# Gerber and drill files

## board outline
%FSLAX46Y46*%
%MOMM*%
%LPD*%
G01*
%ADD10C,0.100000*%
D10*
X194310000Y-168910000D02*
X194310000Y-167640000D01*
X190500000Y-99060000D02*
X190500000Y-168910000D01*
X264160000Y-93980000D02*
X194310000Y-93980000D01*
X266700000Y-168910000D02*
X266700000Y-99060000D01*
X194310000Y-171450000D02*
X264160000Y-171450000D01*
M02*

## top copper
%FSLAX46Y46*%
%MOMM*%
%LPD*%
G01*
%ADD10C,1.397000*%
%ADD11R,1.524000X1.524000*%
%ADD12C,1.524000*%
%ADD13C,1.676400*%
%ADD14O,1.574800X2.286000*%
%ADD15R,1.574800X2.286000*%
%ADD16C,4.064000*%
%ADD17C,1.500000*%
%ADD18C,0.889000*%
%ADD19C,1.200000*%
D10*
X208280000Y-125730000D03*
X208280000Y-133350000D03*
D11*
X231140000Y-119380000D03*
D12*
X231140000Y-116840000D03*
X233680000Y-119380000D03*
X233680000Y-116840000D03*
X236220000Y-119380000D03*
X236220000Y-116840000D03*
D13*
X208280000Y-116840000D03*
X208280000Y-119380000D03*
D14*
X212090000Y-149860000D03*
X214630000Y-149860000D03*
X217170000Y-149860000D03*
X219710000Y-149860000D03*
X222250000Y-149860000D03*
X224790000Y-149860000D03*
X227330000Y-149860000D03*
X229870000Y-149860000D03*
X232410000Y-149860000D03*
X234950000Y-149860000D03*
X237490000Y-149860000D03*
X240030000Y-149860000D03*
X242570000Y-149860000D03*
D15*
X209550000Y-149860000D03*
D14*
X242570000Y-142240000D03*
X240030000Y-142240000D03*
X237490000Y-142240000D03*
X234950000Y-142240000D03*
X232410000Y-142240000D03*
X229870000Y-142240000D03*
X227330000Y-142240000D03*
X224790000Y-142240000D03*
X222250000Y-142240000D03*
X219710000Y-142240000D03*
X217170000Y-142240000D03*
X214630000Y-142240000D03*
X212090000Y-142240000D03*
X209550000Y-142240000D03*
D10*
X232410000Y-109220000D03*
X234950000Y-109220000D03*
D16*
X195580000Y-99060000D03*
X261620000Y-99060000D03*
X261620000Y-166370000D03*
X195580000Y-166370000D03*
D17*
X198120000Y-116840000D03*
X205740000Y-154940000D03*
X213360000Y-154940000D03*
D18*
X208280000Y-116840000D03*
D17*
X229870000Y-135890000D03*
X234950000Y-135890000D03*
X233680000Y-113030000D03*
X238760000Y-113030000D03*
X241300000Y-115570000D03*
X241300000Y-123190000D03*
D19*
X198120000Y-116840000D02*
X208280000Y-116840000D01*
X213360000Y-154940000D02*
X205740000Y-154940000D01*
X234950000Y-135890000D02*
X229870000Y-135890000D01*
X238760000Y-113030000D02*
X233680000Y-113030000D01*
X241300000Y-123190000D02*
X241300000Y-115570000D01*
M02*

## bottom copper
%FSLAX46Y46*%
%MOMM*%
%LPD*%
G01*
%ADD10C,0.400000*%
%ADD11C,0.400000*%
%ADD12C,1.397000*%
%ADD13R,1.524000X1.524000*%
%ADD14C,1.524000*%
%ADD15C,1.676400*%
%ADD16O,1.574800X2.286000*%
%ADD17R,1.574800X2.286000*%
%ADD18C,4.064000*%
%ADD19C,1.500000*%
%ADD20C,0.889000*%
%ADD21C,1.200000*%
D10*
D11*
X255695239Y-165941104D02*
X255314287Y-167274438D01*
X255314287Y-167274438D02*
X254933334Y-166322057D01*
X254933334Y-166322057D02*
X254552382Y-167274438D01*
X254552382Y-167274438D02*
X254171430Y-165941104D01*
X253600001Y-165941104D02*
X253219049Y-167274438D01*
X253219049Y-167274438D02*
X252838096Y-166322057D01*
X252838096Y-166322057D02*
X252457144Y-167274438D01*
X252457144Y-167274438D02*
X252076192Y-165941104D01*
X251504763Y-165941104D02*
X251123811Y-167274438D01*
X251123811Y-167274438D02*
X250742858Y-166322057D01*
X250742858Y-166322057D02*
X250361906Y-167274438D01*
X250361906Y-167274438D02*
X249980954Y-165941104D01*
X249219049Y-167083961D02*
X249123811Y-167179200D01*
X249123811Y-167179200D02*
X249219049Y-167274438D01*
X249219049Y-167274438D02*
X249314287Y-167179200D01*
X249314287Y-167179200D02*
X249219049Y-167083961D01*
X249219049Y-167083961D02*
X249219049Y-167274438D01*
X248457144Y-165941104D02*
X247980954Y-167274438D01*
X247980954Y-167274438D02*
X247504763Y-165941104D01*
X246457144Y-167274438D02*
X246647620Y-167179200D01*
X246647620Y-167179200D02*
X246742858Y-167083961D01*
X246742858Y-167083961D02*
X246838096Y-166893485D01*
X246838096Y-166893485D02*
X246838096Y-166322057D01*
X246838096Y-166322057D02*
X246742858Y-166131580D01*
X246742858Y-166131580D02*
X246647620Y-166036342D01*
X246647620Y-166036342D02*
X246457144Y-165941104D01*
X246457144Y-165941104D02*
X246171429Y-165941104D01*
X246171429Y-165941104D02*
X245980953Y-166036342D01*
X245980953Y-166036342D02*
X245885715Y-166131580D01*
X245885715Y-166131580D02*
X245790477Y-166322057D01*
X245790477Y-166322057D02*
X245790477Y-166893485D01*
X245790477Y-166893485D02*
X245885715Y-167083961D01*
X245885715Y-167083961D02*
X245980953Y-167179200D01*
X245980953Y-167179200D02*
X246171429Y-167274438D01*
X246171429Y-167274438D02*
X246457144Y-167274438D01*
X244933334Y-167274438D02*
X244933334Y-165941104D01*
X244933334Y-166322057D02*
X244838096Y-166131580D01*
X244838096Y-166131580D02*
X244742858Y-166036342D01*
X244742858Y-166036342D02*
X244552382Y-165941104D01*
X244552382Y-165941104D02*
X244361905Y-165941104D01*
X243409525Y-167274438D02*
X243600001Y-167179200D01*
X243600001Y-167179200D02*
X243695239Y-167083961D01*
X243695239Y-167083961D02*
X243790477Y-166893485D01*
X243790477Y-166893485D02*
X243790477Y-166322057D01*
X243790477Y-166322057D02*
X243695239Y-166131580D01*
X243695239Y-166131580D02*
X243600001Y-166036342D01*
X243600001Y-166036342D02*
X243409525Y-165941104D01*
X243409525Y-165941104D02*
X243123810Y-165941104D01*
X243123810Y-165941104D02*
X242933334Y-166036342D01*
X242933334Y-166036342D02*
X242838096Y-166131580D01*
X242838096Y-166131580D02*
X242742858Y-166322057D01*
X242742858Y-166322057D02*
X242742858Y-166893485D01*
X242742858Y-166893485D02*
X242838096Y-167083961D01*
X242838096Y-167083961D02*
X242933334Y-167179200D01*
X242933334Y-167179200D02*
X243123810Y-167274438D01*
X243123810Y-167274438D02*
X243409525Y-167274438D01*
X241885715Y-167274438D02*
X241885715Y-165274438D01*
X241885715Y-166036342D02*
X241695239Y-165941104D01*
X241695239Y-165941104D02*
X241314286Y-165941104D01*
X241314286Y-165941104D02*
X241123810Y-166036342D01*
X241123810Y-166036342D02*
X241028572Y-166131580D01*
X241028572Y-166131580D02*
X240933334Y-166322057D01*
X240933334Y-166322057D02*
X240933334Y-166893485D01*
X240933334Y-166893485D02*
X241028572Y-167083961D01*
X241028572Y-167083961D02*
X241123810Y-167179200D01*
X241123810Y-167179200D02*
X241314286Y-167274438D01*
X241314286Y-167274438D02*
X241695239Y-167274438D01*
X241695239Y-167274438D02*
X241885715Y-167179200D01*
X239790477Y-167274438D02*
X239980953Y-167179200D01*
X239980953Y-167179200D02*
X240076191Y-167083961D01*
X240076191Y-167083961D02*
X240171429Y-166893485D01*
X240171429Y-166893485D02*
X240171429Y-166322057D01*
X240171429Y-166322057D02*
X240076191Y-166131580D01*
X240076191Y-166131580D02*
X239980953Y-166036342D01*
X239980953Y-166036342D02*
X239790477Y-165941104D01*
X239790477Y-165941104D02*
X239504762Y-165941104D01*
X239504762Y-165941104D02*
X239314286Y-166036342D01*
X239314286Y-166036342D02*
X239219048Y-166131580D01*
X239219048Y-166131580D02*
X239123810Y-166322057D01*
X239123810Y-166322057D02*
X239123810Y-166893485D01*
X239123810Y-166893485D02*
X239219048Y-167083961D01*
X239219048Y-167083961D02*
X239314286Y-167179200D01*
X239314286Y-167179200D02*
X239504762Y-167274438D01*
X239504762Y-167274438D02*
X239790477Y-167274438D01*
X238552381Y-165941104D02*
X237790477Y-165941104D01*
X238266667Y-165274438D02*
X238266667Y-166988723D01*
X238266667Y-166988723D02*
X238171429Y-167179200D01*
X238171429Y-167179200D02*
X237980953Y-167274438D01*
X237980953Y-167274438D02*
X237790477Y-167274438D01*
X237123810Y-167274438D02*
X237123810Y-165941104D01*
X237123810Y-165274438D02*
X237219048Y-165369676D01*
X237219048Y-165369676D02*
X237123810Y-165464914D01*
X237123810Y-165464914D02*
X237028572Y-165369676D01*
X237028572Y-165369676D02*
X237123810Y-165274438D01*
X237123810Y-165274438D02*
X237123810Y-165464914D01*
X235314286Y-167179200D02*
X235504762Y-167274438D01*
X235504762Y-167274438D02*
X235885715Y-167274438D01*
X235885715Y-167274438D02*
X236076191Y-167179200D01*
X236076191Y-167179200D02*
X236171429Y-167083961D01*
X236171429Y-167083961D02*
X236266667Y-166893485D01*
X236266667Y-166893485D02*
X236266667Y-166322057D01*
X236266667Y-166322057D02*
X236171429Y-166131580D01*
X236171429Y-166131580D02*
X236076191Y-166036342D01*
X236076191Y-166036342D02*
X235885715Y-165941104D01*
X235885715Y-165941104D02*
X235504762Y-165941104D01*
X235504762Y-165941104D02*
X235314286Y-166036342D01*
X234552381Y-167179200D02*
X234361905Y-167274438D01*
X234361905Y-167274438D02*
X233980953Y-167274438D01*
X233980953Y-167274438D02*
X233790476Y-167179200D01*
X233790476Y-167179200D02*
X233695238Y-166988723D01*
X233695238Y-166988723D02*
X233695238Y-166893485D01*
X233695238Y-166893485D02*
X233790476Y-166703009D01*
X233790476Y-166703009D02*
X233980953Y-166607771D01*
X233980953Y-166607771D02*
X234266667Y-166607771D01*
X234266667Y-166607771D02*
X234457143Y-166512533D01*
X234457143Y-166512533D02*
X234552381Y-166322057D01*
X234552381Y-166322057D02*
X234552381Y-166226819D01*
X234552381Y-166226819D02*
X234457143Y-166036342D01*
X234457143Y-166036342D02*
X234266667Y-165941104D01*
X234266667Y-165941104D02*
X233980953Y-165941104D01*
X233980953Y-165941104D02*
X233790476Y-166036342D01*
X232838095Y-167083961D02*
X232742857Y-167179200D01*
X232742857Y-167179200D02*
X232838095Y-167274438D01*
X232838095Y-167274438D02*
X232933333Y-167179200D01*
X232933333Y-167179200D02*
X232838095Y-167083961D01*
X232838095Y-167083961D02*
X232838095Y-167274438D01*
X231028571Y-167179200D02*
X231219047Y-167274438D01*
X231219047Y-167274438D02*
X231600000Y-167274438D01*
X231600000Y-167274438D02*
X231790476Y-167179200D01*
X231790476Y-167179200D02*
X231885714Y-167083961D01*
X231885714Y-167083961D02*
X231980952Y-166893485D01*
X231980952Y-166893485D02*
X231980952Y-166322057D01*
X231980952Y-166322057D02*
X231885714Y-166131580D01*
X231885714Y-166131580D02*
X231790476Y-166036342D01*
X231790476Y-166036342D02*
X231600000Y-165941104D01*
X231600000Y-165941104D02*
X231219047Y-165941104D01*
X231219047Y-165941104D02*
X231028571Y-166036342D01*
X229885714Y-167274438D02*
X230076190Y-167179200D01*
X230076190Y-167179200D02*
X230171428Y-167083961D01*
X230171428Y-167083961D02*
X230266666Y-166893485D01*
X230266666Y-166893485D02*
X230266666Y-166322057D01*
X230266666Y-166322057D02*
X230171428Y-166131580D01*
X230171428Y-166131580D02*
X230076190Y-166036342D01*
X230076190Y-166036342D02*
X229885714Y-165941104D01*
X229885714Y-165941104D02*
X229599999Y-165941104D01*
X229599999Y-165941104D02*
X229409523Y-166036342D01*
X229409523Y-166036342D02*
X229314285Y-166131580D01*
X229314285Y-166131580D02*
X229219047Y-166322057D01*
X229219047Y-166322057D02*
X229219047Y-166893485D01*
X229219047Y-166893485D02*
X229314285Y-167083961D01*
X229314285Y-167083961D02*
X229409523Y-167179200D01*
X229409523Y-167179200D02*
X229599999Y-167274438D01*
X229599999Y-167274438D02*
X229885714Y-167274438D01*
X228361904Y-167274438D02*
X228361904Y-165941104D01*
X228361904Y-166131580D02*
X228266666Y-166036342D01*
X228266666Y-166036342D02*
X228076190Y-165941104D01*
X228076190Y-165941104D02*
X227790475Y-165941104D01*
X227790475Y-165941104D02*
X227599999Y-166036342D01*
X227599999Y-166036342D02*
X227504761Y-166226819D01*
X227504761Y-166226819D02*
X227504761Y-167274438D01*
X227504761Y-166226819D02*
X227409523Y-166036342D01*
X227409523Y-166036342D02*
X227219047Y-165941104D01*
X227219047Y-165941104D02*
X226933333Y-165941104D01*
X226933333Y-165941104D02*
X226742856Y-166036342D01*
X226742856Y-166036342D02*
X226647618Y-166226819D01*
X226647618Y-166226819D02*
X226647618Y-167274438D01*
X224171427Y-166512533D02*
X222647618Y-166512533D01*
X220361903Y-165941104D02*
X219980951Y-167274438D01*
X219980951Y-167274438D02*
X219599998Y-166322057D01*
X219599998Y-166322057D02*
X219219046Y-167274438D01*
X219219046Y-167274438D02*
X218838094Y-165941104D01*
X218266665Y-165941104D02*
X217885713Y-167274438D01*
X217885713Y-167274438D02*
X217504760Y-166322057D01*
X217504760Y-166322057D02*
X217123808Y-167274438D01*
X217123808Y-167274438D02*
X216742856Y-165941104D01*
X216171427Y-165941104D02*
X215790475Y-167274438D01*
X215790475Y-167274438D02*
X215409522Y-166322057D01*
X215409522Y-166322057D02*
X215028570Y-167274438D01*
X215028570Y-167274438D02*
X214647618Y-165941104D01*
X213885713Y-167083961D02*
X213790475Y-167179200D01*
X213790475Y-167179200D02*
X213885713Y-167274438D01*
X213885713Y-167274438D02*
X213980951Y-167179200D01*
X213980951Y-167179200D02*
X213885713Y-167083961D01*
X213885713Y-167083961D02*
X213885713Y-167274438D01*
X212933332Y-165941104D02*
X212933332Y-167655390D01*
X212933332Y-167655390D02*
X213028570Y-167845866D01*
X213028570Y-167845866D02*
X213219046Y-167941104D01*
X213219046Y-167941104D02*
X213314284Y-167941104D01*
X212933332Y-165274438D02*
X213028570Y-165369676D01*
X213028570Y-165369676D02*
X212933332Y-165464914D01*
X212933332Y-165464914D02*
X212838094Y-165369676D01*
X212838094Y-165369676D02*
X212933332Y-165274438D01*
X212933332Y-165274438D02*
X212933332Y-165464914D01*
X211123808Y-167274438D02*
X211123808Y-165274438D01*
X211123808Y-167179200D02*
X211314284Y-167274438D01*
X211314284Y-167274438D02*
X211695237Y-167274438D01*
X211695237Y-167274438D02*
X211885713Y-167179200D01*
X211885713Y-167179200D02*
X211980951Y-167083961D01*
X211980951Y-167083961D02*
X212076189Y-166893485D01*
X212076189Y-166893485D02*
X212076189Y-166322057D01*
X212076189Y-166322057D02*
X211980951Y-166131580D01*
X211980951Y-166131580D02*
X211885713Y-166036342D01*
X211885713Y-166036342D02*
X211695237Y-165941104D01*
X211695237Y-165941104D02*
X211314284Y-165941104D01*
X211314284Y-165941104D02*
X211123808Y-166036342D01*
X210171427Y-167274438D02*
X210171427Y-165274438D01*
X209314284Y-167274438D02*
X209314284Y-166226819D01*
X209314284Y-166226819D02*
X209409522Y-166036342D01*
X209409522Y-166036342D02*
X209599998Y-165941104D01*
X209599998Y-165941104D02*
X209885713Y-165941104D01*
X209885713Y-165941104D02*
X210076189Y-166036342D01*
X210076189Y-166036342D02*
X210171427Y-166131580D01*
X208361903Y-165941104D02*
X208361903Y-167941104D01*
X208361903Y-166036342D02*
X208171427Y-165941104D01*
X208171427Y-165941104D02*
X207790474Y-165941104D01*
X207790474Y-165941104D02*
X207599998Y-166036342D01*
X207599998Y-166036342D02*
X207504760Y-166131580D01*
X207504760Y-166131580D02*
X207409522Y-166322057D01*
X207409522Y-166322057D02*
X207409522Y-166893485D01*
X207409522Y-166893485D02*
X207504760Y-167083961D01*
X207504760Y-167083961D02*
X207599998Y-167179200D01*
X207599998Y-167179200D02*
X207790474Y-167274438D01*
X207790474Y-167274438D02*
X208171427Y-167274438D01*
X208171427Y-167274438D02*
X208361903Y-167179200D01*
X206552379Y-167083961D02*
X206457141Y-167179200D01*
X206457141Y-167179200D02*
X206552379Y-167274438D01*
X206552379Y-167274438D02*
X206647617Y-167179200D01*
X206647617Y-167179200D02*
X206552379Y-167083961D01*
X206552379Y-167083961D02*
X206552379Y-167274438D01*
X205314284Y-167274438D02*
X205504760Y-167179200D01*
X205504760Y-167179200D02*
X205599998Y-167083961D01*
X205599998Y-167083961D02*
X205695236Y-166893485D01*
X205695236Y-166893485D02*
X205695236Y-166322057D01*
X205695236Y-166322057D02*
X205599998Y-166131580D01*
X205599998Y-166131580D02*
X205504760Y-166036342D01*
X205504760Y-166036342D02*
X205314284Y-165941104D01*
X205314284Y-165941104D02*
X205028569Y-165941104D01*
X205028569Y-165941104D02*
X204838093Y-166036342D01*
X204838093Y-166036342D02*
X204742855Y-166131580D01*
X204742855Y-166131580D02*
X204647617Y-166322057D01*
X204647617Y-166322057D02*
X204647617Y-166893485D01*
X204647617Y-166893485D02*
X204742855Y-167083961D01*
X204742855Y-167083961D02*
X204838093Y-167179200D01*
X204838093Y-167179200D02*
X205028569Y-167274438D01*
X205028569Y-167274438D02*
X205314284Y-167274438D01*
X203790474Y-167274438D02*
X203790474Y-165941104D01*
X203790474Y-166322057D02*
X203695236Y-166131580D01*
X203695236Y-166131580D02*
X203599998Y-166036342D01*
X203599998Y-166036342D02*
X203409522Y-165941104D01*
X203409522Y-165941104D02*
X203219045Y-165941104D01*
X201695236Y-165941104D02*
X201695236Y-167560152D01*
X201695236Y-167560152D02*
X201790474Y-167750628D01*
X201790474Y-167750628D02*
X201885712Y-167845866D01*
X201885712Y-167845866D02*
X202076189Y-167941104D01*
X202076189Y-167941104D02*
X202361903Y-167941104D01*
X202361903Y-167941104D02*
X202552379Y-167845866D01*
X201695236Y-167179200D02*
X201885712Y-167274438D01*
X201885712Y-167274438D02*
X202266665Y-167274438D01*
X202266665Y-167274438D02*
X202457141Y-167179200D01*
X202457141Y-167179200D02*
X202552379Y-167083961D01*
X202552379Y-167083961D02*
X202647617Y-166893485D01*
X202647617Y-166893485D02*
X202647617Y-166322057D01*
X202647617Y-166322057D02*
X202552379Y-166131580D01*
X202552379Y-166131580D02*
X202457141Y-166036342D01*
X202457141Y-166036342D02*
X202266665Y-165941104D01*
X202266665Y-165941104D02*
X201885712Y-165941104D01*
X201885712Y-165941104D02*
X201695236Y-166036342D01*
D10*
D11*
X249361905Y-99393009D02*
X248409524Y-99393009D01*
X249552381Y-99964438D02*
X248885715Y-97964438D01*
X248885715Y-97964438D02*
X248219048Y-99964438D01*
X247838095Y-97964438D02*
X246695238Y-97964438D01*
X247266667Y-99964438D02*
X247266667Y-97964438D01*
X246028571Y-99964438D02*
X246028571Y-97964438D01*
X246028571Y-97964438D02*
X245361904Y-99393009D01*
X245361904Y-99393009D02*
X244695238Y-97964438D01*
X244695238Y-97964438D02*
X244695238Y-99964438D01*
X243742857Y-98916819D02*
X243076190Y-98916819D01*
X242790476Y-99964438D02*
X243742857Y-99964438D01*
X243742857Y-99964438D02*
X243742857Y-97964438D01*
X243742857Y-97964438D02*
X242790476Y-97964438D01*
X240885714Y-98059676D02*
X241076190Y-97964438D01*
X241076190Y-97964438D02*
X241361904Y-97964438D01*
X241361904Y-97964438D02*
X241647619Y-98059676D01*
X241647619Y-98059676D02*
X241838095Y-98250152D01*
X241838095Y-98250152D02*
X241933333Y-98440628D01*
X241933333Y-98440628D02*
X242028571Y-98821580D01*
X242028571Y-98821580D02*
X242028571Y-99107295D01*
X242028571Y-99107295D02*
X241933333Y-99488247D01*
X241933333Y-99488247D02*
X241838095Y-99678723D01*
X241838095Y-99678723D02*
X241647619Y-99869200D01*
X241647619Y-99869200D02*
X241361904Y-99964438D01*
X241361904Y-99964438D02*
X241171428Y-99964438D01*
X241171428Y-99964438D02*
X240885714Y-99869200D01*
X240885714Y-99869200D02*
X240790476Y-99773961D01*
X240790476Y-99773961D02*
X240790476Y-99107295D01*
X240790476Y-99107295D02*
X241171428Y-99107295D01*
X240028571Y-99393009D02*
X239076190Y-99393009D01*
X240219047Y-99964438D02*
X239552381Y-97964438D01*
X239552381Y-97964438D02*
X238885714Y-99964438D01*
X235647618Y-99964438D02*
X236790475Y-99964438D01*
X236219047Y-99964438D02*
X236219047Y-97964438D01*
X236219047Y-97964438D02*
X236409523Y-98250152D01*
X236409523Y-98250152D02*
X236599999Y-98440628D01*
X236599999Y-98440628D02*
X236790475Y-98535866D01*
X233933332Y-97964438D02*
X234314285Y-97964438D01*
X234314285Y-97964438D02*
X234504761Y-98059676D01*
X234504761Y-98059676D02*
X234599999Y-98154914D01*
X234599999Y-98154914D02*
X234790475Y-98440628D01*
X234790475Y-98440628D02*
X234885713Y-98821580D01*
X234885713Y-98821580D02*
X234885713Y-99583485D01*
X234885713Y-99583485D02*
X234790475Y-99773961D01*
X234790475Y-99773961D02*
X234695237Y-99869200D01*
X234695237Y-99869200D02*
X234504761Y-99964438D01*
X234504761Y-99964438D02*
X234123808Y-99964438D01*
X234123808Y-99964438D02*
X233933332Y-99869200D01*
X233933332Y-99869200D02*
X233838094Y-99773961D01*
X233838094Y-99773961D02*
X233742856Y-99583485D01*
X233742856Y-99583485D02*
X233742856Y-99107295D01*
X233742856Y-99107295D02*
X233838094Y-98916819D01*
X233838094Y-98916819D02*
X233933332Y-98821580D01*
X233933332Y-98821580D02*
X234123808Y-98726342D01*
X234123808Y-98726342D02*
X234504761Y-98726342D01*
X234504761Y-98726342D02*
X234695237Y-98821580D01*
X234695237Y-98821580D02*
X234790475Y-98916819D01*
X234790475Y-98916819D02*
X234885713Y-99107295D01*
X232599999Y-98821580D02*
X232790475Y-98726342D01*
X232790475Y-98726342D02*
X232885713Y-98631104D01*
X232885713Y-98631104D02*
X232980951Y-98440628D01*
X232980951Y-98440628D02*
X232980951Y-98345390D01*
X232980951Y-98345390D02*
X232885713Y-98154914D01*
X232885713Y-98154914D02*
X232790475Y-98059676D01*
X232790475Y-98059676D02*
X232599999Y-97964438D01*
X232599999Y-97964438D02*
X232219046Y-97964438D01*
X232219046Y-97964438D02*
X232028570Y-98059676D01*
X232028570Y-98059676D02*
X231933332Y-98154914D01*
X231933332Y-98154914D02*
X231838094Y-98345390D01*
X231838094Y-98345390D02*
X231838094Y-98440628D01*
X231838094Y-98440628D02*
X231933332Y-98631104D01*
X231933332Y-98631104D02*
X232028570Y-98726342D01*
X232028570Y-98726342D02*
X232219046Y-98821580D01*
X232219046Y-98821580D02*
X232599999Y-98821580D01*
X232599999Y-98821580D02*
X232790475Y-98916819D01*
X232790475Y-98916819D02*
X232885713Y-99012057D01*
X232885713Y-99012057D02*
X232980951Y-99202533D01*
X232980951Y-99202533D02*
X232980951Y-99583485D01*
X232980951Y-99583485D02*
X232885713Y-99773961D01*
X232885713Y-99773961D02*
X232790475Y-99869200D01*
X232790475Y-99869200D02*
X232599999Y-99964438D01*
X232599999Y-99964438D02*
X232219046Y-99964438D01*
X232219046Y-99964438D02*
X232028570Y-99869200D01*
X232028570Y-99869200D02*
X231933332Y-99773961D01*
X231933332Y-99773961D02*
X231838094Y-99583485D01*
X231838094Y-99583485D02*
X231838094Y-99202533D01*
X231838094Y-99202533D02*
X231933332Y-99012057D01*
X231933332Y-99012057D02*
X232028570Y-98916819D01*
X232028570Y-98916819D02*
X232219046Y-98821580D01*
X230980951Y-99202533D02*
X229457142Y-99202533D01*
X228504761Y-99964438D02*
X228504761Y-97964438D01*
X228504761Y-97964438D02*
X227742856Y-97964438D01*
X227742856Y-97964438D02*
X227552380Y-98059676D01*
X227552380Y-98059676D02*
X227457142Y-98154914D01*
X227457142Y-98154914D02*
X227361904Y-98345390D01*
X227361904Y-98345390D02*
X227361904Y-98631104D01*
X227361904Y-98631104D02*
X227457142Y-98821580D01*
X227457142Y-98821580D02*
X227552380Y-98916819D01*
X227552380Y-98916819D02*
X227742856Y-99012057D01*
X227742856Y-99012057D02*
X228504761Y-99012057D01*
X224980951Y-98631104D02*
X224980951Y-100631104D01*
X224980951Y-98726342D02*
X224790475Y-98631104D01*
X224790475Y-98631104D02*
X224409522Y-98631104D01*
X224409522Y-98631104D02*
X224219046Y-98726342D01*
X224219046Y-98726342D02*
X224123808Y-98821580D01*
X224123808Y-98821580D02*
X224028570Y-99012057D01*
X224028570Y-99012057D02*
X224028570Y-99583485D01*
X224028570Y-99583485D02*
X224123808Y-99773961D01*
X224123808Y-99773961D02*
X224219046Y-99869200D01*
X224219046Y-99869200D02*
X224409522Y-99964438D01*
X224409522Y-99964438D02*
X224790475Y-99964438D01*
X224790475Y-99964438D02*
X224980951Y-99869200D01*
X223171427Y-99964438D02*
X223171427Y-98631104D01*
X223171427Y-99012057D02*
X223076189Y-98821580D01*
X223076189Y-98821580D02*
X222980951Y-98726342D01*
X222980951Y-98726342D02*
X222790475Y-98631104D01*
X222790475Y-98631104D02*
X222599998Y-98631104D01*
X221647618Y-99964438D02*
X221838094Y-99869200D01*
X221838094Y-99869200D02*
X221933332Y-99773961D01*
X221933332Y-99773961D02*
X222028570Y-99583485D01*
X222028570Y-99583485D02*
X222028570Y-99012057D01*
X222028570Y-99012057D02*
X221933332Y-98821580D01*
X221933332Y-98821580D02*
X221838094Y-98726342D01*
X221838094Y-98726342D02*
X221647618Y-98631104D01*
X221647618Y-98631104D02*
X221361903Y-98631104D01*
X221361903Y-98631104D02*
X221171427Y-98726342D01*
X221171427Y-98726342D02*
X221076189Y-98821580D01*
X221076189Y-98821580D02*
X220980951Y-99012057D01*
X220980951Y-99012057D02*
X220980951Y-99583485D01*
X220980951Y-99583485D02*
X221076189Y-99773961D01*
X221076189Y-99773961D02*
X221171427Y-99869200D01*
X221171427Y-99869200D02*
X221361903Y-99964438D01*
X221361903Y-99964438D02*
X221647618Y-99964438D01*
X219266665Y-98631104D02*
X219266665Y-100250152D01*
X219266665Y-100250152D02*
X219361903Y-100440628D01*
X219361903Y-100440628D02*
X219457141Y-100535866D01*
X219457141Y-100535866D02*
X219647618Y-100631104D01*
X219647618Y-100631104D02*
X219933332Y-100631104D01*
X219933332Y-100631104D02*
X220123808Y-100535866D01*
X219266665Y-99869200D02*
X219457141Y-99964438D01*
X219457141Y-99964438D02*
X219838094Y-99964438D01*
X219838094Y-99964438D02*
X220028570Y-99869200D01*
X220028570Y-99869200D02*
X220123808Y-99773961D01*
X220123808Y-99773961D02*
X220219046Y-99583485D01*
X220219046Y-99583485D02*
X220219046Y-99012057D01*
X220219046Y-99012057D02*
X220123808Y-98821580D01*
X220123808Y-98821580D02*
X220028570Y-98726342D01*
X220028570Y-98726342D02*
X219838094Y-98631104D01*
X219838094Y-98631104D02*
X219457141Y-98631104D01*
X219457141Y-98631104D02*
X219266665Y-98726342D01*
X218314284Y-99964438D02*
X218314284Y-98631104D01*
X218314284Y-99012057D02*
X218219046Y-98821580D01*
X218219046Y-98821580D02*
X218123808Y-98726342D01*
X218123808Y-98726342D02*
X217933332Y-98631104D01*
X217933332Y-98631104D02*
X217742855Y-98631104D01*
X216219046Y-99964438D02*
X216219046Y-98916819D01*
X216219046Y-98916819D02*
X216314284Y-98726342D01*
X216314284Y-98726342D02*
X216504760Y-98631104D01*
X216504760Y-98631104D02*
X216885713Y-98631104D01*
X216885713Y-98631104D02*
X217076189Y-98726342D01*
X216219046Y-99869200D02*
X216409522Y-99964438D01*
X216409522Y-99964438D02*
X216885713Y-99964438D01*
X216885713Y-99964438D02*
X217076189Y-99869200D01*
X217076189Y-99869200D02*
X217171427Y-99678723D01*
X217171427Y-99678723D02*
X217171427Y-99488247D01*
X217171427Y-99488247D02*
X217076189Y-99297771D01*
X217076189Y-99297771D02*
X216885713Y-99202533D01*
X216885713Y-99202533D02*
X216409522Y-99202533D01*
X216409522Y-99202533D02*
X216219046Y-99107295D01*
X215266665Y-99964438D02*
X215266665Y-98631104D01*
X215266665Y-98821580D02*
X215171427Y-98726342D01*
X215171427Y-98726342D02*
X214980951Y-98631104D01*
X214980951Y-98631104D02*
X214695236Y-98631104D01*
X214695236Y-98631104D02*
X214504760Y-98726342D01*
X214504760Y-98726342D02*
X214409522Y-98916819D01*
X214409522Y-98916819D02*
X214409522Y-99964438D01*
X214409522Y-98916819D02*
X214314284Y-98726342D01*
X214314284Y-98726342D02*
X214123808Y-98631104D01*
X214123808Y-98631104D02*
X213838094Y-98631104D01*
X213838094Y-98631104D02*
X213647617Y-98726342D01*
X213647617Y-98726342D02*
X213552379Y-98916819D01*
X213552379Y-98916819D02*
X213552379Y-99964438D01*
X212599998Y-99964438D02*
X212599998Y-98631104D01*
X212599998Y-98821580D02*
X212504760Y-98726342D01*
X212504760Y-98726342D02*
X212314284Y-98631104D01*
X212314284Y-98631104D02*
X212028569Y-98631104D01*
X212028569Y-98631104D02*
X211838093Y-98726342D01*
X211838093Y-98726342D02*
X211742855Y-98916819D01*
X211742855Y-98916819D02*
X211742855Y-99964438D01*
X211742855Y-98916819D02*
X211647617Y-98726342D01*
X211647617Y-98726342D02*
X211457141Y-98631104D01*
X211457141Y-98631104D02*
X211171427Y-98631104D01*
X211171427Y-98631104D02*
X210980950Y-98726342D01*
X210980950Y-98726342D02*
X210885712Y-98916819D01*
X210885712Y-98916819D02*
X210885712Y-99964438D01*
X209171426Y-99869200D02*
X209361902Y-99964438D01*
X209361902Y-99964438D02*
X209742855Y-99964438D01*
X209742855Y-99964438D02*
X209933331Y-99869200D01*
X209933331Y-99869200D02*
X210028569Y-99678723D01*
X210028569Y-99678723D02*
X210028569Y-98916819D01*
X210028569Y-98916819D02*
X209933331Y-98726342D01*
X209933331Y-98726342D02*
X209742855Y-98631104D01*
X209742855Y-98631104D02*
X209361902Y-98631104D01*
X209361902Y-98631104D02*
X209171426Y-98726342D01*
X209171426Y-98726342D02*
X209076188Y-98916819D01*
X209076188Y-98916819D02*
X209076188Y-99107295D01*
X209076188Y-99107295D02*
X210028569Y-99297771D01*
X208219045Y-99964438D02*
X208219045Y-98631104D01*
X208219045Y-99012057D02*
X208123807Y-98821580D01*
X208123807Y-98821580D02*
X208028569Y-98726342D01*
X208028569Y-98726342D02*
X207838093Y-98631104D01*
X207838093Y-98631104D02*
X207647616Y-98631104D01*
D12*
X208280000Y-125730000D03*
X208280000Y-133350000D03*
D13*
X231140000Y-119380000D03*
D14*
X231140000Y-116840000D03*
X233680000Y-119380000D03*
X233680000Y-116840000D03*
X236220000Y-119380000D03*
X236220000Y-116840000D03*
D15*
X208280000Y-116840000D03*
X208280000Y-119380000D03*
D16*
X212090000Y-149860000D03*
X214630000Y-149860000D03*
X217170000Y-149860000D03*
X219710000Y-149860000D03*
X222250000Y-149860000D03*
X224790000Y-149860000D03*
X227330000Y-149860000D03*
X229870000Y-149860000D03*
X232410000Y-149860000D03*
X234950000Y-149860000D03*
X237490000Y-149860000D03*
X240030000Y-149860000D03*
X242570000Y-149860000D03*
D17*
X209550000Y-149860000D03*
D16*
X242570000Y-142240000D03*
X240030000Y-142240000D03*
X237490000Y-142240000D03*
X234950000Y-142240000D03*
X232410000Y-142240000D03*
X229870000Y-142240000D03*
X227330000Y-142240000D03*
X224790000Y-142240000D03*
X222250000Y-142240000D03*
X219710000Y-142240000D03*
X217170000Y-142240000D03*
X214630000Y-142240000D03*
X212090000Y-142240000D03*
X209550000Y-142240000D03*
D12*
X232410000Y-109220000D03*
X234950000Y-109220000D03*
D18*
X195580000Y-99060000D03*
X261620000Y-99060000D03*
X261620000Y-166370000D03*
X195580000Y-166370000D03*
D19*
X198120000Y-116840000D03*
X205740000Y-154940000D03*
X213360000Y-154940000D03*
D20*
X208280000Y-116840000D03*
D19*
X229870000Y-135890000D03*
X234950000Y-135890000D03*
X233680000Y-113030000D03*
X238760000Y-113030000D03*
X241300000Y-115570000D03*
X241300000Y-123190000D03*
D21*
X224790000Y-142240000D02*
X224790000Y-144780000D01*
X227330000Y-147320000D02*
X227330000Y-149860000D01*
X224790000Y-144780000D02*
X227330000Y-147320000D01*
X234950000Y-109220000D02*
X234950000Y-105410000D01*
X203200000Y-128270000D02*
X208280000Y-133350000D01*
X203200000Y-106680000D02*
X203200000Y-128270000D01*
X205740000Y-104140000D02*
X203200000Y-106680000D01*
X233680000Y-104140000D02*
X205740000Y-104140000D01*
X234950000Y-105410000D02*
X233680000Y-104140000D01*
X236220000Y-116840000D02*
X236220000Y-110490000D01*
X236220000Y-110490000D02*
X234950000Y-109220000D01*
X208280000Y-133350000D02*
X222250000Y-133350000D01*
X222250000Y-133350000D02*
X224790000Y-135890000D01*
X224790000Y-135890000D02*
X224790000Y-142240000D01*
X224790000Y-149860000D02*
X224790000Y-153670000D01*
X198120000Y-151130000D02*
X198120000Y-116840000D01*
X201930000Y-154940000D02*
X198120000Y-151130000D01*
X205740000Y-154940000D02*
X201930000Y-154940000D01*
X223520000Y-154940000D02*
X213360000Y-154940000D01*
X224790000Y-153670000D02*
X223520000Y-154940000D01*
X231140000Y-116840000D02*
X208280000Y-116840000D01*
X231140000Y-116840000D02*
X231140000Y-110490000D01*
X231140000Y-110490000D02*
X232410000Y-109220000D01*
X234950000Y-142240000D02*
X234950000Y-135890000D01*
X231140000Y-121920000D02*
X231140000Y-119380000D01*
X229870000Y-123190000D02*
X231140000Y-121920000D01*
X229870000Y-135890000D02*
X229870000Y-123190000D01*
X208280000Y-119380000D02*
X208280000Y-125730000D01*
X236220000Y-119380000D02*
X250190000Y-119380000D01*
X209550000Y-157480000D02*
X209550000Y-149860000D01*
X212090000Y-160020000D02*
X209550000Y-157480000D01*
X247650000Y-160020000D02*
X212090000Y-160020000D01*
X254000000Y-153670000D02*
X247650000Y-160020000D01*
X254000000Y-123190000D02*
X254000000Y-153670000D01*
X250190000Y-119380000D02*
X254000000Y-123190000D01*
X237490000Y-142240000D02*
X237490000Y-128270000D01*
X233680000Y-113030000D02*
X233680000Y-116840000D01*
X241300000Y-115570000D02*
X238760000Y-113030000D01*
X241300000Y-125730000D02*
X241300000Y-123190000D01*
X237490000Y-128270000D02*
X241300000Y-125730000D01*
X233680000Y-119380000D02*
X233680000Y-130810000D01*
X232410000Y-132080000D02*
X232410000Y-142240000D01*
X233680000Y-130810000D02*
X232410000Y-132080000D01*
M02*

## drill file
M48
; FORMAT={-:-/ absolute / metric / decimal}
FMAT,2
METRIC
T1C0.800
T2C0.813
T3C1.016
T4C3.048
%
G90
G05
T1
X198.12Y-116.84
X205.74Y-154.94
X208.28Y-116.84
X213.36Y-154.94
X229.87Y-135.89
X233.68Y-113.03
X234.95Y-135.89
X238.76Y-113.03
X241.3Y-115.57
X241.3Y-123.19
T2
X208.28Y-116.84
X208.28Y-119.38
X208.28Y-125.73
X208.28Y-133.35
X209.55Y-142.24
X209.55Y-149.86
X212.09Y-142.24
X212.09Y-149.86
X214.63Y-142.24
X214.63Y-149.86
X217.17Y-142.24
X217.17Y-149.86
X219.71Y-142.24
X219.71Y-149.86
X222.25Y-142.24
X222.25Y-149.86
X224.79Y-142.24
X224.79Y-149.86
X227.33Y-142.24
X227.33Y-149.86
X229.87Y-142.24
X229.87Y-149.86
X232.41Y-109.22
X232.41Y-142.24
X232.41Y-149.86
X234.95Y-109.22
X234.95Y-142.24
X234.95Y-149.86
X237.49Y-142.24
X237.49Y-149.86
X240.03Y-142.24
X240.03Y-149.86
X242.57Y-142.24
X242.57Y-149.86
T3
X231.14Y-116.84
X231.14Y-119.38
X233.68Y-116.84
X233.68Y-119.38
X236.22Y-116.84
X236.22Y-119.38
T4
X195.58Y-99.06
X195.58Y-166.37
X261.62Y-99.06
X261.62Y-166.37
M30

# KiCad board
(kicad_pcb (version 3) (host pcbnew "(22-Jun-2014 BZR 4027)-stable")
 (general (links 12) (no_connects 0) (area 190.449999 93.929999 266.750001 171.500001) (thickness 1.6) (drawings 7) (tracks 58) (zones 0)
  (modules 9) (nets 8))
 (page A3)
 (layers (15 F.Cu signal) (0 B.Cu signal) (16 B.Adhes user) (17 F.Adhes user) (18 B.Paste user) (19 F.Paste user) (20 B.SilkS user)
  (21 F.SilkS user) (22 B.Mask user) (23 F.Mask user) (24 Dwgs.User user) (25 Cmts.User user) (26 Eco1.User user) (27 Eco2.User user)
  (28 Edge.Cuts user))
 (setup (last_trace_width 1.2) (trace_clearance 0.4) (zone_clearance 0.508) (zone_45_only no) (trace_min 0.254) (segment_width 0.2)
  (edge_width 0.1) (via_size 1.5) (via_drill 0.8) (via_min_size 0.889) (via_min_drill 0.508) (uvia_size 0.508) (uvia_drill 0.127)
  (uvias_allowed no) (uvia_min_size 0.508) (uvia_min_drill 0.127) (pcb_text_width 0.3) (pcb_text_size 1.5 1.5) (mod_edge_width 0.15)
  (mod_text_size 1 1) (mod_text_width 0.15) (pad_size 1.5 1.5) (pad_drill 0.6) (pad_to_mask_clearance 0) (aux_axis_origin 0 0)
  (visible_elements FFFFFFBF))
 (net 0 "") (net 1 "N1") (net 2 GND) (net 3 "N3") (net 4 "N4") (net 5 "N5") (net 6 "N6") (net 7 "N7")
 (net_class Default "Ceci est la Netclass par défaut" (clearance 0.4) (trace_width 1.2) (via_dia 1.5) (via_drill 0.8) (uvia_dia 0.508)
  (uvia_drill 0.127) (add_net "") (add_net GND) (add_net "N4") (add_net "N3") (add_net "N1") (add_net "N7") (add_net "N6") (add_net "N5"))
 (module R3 (layer F.Cu) (at 208.28 129.54 270) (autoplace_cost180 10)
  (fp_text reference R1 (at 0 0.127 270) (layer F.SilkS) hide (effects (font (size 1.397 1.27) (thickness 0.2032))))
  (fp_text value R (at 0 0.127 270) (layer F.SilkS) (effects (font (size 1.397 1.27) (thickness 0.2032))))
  (pad 1 thru_hole circle (at -3.81 0 270) (size 1.397 1.397) (drill 0.8128) (layers *.Cu *.Mask F.SilkS) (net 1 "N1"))
  (pad 2 thru_hole circle (at 3.81 0 270) (size 1.397 1.397) (drill 0.8128) (layers *.Cu *.Mask F.SilkS) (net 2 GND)))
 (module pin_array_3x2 (layer F.Cu) (at 233.68 118.11)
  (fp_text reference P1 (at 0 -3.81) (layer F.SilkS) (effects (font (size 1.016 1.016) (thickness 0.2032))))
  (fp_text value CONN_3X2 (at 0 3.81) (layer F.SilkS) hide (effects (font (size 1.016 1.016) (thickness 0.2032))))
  (pad 1 thru_hole rect (at -2.54 1.27) (size 1.524 1.524) (drill 1.016) (layers *.Cu *.Mask F.SilkS) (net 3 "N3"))
  (pad 2 thru_hole circle (at -2.54 -1.27) (size 1.524 1.524) (drill 1.016) (layers *.Cu *.Mask F.SilkS) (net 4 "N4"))
  (pad 3 thru_hole circle (at 0 1.27) (size 1.524 1.524) (drill 1.016) (layers *.Cu *.Mask F.SilkS) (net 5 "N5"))
  (pad 4 thru_hole circle (at 0 -1.27) (size 1.524 1.524) (drill 1.016) (layers *.Cu *.Mask F.SilkS) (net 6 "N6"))
  (pad 5 thru_hole circle (at 2.54 1.27) (size 1.524 1.524) (drill 1.016) (layers *.Cu *.Mask F.SilkS) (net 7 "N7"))
  (pad 6 thru_hole circle (at 2.54 -1.27) (size 1.524 1.524) (drill 1.016) (layers *.Cu *.Mask F.SilkS) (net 2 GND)))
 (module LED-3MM (layer F.Cu) (at 208.28 118.11 270)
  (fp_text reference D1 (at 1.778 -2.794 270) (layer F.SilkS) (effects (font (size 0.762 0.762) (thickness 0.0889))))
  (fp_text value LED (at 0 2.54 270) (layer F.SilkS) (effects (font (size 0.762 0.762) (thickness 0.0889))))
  (pad 1 thru_hole circle (at -1.27 0 270) (size 1.6764 1.6764) (drill 0.8128) (layers *.Cu *.Mask F.SilkS) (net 4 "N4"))
  (pad 2 thru_hole circle (at 1.27 0 270) (size 1.6764 1.6764) (drill 0.8128) (layers *.Cu *.Mask F.SilkS) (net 1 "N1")))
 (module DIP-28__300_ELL (layer F.Cu) (at 226.06 146.05)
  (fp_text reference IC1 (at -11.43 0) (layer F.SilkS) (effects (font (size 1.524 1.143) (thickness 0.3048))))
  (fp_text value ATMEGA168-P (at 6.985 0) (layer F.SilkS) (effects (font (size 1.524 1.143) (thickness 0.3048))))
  (pad 2 thru_hole oval (at -13.97 3.81) (size 1.5748 2.286) (drill 0.8128) (layers *.Cu *.Mask F.SilkS))
  (pad 3 thru_hole oval (at -11.43 3.81) (size 1.5748 2.286) (drill 0.8128) (layers *.Cu *.Mask F.SilkS))
  (pad 4 thru_hole oval (at -8.89 3.81) (size 1.5748 2.286) (drill 0.8128) (layers *.Cu *.Mask F.SilkS))
  (pad 5 thru_hole oval (at -6.35 3.81) (size 1.5748 2.286) (drill 0.8128) (layers *.Cu *.Mask F.SilkS))
  (pad 6 thru_hole oval (at -3.81 3.81) (size 1.5748 2.286) (drill 0.8128) (layers *.Cu *.Mask F.SilkS))
  (pad 7 thru_hole oval (at -1.27 3.81) (size 1.5748 2.286) (drill 0.8128) (layers *.Cu *.Mask F.SilkS) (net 4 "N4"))
  (pad 8 thru_hole oval (at 1.27 3.81) (size 1.5748 2.286) (drill 0.8128) (layers *.Cu *.Mask F.SilkS) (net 2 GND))
  (pad 9 thru_hole oval (at 3.81 3.81) (size 1.5748 2.286) (drill 0.8128) (layers *.Cu *.Mask F.SilkS))
  (pad 10 thru_hole oval (at 6.35 3.81) (size 1.5748 2.286) (drill 0.8128) (layers *.Cu *.Mask F.SilkS))
  (pad 11 thru_hole oval (at 8.89 3.81) (size 1.5748 2.286) (drill 0.8128) (layers *.Cu *.Mask F.SilkS))
  (pad 12 thru_hole oval (at 11.43 3.81) (size 1.5748 2.286) (drill 0.8128) (layers *.Cu *.Mask F.SilkS))
  (pad 13 thru_hole oval (at 13.97 3.81) (size 1.5748 2.286) (drill 0.8128) (layers *.Cu *.Mask F.SilkS))
  (pad 14 thru_hole oval (at 16.51 3.81) (size 1.5748 2.286) (drill 0.8128) (layers *.Cu *.Mask F.SilkS))
  (pad 1 thru_hole rect (at -16.51 3.81) (size 1.5748 2.286) (drill 0.8128) (layers *.Cu *.Mask F.SilkS) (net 7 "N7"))
  (pad 15 thru_hole oval (at 16.51 -3.81) (size 1.5748 2.286) (drill 0.8128) (layers *.Cu *.Mask F.SilkS))
  (pad 16 thru_hole oval (at 13.97 -3.81) (size 1.5748 2.286) (drill 0.8128) (layers *.Cu *.Mask F.SilkS))
  (pad 17 thru_hole oval (at 11.43 -3.81) (size 1.5748 2.286) (drill 0.8128) (layers *.Cu *.Mask F.SilkS) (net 6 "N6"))
  (pad 18 thru_hole oval (at 8.89 -3.81) (size 1.5748 2.286) (drill 0.8128) (layers *.Cu *.Mask F.SilkS) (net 3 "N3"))
  (pad 19 thru_hole oval (at 6.35 -3.81) (size 1.5748 2.286) (drill 0.8128) (layers *.Cu *.Mask F.SilkS) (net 5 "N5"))
  (pad 20 thru_hole oval (at 3.81 -3.81) (size 1.5748 2.286) (drill 0.8128) (layers *.Cu *.Mask F.SilkS))
  (pad 21 thru_hole oval (at 1.27 -3.81) (size 1.5748 2.286) (drill 0.8128) (layers *.Cu *.Mask F.SilkS))
  (pad 22 thru_hole oval (at -1.27 -3.81) (size 1.5748 2.286) (drill 0.8128) (layers *.Cu *.Mask F.SilkS) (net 2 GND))
  (pad 23 thru_hole oval (at -3.81 -3.81) (size 1.5748 2.286) (drill 0.8128) (layers *.Cu *.Mask F.SilkS))
  (pad 24 thru_hole oval (at -6.35 -3.81) (size 1.5748 2.286) (drill 0.8128) (layers *.Cu *.Mask F.SilkS))
  (pad 25 thru_hole oval (at -8.89 -3.81) (size 1.5748 2.286) (drill 0.8128) (layers *.Cu *.Mask F.SilkS))
  (pad 26 thru_hole oval (at -11.43 -3.81) (size 1.5748 2.286) (drill 0.8128) (layers *.Cu *.Mask F.SilkS))
  (pad 27 thru_hole oval (at -13.97 -3.81) (size 1.5748 2.286) (drill 0.8128) (layers *.Cu *.Mask F.SilkS))
  (pad 28 thru_hole oval (at -16.51 -3.81) (size 1.5748 2.286) (drill 0.8128) (layers *.Cu *.Mask F.SilkS)))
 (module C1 (layer F.Cu) (at 233.68 109.22)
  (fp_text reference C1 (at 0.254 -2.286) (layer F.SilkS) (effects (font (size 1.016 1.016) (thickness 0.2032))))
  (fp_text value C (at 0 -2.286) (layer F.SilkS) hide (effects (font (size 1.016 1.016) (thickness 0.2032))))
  (pad 1 thru_hole circle (at -1.27 0) (size 1.397 1.397) (drill 0.8128) (layers *.Cu *.Mask F.SilkS) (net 4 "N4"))
  (pad 2 thru_hole circle (at 1.27 0) (size 1.397 1.397) (drill 0.8128) (layers *.Cu *.Mask F.SilkS) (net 2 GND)))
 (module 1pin (layer F.Cu) (at 195.58 99.06)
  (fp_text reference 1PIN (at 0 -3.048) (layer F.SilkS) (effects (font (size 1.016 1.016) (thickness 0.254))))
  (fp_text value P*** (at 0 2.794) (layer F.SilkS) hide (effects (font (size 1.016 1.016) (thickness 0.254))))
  (pad 1 thru_hole circle (at 0 0) (size 4.064 4.064) (drill 3.048) (layers *.Cu *.Mask F.SilkS)))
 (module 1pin (layer F.Cu) (at 261.62 99.06)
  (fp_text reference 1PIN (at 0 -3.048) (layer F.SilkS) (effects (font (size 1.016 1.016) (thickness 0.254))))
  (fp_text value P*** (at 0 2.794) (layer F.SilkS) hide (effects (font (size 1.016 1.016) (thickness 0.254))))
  (pad 1 thru_hole circle (at 0 0) (size 4.064 4.064) (drill 3.048) (layers *.Cu *.Mask F.SilkS)))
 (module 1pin (layer F.Cu) (at 261.62 166.37)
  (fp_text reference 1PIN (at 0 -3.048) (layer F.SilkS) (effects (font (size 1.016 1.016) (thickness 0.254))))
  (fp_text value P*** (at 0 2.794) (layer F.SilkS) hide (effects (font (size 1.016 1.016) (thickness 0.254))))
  (pad 1 thru_hole circle (at 0 0) (size 4.064 4.064) (drill 3.048) (layers *.Cu *.Mask F.SilkS)))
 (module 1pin (layer F.Cu) (at 195.58 166.37)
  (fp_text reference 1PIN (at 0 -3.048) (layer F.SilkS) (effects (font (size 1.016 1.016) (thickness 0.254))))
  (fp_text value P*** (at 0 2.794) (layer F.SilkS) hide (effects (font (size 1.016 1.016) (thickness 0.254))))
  (pad 1 thru_hole circle (at 0 0) (size 4.064 4.064) (drill 3.048) (layers *.Cu *.Mask F.SilkS)))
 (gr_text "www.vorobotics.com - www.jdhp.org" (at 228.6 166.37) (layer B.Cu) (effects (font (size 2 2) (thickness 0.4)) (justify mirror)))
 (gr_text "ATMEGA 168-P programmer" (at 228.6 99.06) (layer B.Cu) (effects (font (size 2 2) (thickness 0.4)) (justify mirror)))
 (gr_line (start 194.31 168.91) (end 194.31 167.64) (angle 90) (layer Edge.Cuts) (width 0.1))
 (gr_line (start 190.5 99.06) (end 190.5 168.91) (angle 90) (layer Edge.Cuts) (width 0.1))
 (gr_line (start 264.16 93.98) (end 194.31 93.98) (angle 90) (layer Edge.Cuts) (width 0.1))
 (gr_line (start 266.7 168.91) (end 266.7 99.06) (angle 90) (layer Edge.Cuts) (width 0.1))
 (gr_line (start 194.31 171.45) (end 264.16 171.45) (angle 90) (layer Edge.Cuts) (width 0.1))
 (segment (start 224.79 142.24) (end 224.79 144.78) (width 1.2) (layer B.Cu) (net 2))
 (segment (start 227.33 147.32) (end 227.33 149.86) (width 1.2) (layer B.Cu) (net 2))
 (segment (start 224.79 144.78) (end 227.33 147.32) (width 1.2) (layer B.Cu) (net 2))
 (segment (start 234.95 109.22) (end 234.95 105.41) (width 1.2) (layer B.Cu) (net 2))
 (segment (start 203.2 128.27) (end 208.28 133.35) (width 1.2) (layer B.Cu) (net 2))
 (segment (start 203.2 106.68) (end 203.2 128.27) (width 1.2) (layer B.Cu) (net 2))
 (segment (start 205.74 104.14) (end 203.2 106.68) (width 1.2) (layer B.Cu) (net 2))
 (segment (start 233.68 104.14) (end 205.74 104.14) (width 1.2) (layer B.Cu) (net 2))
 (segment (start 234.95 105.41) (end 233.68 104.14) (width 1.2) (layer B.Cu) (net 2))
 (segment (start 236.22 116.84) (end 236.22 110.49) (width 1.2) (layer B.Cu) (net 2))
 (segment (start 236.22 110.49) (end 234.95 109.22) (width 1.2) (layer B.Cu) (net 2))
 (segment (start 208.28 133.35) (end 222.25 133.35) (width 1.2) (layer B.Cu) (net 2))
 (segment (start 222.25 133.35) (end 224.79 135.89) (width 1.2) (layer B.Cu) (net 2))
 (segment (start 224.79 135.89) (end 224.79 142.24) (width 1.2) (layer B.Cu) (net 2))
 (segment (start 224.79 149.86) (end 224.79 153.67) (width 1.2) (layer B.Cu) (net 4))
 (segment (start 198.12 116.84) (end 208.28 116.84) (width 1.2) (layer F.Cu) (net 4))
 (via (at 198.12 116.84) (size 1.5) (layers F.Cu B.Cu) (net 4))
 (segment (start 198.12 151.13) (end 198.12 116.84) (width 1.2) (layer B.Cu) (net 4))
 (segment (start 201.93 154.94) (end 198.12 151.13) (width 1.2) (layer B.Cu) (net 4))
 (segment (start 205.74 154.94) (end 201.93 154.94) (width 1.2) (layer B.Cu) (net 4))
 (via (at 205.74 154.94) (size 1.5) (layers F.Cu B.Cu) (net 4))
 (segment (start 213.36 154.94) (end 205.74 154.94) (width 1.2) (layer F.Cu) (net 4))
 (via (at 213.36 154.94) (size 1.5) (layers F.Cu B.Cu) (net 4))
 (segment (start 223.52 154.94) (end 213.36 154.94) (width 1.2) (layer B.Cu) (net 4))
 (segment (start 224.79 153.67) (end 223.52 154.94) (width 1.2) (layer B.Cu) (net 4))
 (via (at 208.28 116.84) (size 0.889) (layers F.Cu B.Cu) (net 4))
 (segment (start 231.14 116.84) (end 208.28 116.84) (width 1.2) (layer B.Cu) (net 4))
 (segment (start 231.14 116.84) (end 231.14 110.49) (width 1.2) (layer B.Cu) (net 4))
 (segment (start 231.14 110.49) (end 232.41 109.22) (width 1.2) (layer B.Cu) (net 4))
 (segment (start 234.95 142.24) (end 234.95 135.89) (width 1.2) (layer B.Cu) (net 3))
 (segment (start 231.14 121.92) (end 231.14 119.38) (width 1.2) (layer B.Cu) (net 3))
 (segment (start 229.87 123.19) (end 231.14 121.92) (width 1.2) (layer B.Cu) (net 3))
 (segment (start 229.87 135.89) (end 229.87 123.19) (width 1.2) (layer B.Cu) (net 3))
 (via (at 229.87 135.89) (size 1.5) (layers F.Cu B.Cu) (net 3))
 (segment (start 234.95 135.89) (end 229.87 135.89) (width 1.2) (layer F.Cu) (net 3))
 (via (at 234.95 135.89) (size 1.5) (layers F.Cu B.Cu) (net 3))
 (segment (start 208.28 119.38) (end 208.28 125.73) (width 1.2) (layer B.Cu) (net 1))
 (segment (start 236.22 119.38) (end 250.19 119.38) (width 1.2) (layer B.Cu) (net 7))
 (segment (start 209.55 157.48) (end 209.55 149.86) (width 1.2) (layer B.Cu) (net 7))
 (segment (start 212.09 160.02) (end 209.55 157.48) (width 1.2) (layer B.Cu) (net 7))
 (segment (start 247.65 160.02) (end 212.09 160.02) (width 1.2) (layer B.Cu) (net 7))
 (segment (start 254 153.67) (end 247.65 160.02) (width 1.2) (layer B.Cu) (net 7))
 (segment (start 254 123.19) (end 254 153.67) (width 1.2) (layer B.Cu) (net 7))
 (segment (start 250.19 119.38) (end 254 123.19) (width 1.2) (layer B.Cu) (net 7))
 (segment (start 237.49 142.24) (end 237.49 128.27) (width 1.2) (layer B.Cu) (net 6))
 (segment (start 233.68 113.03) (end 233.68 116.84) (width 1.2) (layer B.Cu) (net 6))
 (via (at 233.68 113.03) (size 1.5) (layers F.Cu B.Cu) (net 6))
 (segment (start 238.76 113.03) (end 233.68 113.03) (width 1.2) (layer F.Cu) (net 6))
 (via (at 238.76 113.03) (size 1.5) (layers F.Cu B.Cu) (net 6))
 (segment (start 241.3 115.57) (end 238.76 113.03) (width 1.2) (layer B.Cu) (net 6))
 (via (at 241.3 115.57) (size 1.5) (layers F.Cu B.Cu) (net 6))
 (segment (start 241.3 123.19) (end 241.3 115.57) (width 1.2) (layer F.Cu) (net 6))
 (via (at 241.3 123.19) (size 1.5) (layers F.Cu B.Cu) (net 6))
 (segment (start 241.3 125.73) (end 241.3 123.19) (width 1.2) (layer B.Cu) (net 6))
 (segment (start 237.49 128.27) (end 241.3 125.73) (width 1.2) (layer B.Cu) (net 6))
 (segment (start 233.68 119.38) (end 233.68 130.81) (width 1.2) (layer B.Cu) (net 5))
 (segment (start 232.41 132.08) (end 232.41 142.24) (width 1.2) (layer B.Cu) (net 5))
 (segment (start 233.68 130.81) (end 232.41 132.08) (width 1.2) (layer B.Cu) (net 5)))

